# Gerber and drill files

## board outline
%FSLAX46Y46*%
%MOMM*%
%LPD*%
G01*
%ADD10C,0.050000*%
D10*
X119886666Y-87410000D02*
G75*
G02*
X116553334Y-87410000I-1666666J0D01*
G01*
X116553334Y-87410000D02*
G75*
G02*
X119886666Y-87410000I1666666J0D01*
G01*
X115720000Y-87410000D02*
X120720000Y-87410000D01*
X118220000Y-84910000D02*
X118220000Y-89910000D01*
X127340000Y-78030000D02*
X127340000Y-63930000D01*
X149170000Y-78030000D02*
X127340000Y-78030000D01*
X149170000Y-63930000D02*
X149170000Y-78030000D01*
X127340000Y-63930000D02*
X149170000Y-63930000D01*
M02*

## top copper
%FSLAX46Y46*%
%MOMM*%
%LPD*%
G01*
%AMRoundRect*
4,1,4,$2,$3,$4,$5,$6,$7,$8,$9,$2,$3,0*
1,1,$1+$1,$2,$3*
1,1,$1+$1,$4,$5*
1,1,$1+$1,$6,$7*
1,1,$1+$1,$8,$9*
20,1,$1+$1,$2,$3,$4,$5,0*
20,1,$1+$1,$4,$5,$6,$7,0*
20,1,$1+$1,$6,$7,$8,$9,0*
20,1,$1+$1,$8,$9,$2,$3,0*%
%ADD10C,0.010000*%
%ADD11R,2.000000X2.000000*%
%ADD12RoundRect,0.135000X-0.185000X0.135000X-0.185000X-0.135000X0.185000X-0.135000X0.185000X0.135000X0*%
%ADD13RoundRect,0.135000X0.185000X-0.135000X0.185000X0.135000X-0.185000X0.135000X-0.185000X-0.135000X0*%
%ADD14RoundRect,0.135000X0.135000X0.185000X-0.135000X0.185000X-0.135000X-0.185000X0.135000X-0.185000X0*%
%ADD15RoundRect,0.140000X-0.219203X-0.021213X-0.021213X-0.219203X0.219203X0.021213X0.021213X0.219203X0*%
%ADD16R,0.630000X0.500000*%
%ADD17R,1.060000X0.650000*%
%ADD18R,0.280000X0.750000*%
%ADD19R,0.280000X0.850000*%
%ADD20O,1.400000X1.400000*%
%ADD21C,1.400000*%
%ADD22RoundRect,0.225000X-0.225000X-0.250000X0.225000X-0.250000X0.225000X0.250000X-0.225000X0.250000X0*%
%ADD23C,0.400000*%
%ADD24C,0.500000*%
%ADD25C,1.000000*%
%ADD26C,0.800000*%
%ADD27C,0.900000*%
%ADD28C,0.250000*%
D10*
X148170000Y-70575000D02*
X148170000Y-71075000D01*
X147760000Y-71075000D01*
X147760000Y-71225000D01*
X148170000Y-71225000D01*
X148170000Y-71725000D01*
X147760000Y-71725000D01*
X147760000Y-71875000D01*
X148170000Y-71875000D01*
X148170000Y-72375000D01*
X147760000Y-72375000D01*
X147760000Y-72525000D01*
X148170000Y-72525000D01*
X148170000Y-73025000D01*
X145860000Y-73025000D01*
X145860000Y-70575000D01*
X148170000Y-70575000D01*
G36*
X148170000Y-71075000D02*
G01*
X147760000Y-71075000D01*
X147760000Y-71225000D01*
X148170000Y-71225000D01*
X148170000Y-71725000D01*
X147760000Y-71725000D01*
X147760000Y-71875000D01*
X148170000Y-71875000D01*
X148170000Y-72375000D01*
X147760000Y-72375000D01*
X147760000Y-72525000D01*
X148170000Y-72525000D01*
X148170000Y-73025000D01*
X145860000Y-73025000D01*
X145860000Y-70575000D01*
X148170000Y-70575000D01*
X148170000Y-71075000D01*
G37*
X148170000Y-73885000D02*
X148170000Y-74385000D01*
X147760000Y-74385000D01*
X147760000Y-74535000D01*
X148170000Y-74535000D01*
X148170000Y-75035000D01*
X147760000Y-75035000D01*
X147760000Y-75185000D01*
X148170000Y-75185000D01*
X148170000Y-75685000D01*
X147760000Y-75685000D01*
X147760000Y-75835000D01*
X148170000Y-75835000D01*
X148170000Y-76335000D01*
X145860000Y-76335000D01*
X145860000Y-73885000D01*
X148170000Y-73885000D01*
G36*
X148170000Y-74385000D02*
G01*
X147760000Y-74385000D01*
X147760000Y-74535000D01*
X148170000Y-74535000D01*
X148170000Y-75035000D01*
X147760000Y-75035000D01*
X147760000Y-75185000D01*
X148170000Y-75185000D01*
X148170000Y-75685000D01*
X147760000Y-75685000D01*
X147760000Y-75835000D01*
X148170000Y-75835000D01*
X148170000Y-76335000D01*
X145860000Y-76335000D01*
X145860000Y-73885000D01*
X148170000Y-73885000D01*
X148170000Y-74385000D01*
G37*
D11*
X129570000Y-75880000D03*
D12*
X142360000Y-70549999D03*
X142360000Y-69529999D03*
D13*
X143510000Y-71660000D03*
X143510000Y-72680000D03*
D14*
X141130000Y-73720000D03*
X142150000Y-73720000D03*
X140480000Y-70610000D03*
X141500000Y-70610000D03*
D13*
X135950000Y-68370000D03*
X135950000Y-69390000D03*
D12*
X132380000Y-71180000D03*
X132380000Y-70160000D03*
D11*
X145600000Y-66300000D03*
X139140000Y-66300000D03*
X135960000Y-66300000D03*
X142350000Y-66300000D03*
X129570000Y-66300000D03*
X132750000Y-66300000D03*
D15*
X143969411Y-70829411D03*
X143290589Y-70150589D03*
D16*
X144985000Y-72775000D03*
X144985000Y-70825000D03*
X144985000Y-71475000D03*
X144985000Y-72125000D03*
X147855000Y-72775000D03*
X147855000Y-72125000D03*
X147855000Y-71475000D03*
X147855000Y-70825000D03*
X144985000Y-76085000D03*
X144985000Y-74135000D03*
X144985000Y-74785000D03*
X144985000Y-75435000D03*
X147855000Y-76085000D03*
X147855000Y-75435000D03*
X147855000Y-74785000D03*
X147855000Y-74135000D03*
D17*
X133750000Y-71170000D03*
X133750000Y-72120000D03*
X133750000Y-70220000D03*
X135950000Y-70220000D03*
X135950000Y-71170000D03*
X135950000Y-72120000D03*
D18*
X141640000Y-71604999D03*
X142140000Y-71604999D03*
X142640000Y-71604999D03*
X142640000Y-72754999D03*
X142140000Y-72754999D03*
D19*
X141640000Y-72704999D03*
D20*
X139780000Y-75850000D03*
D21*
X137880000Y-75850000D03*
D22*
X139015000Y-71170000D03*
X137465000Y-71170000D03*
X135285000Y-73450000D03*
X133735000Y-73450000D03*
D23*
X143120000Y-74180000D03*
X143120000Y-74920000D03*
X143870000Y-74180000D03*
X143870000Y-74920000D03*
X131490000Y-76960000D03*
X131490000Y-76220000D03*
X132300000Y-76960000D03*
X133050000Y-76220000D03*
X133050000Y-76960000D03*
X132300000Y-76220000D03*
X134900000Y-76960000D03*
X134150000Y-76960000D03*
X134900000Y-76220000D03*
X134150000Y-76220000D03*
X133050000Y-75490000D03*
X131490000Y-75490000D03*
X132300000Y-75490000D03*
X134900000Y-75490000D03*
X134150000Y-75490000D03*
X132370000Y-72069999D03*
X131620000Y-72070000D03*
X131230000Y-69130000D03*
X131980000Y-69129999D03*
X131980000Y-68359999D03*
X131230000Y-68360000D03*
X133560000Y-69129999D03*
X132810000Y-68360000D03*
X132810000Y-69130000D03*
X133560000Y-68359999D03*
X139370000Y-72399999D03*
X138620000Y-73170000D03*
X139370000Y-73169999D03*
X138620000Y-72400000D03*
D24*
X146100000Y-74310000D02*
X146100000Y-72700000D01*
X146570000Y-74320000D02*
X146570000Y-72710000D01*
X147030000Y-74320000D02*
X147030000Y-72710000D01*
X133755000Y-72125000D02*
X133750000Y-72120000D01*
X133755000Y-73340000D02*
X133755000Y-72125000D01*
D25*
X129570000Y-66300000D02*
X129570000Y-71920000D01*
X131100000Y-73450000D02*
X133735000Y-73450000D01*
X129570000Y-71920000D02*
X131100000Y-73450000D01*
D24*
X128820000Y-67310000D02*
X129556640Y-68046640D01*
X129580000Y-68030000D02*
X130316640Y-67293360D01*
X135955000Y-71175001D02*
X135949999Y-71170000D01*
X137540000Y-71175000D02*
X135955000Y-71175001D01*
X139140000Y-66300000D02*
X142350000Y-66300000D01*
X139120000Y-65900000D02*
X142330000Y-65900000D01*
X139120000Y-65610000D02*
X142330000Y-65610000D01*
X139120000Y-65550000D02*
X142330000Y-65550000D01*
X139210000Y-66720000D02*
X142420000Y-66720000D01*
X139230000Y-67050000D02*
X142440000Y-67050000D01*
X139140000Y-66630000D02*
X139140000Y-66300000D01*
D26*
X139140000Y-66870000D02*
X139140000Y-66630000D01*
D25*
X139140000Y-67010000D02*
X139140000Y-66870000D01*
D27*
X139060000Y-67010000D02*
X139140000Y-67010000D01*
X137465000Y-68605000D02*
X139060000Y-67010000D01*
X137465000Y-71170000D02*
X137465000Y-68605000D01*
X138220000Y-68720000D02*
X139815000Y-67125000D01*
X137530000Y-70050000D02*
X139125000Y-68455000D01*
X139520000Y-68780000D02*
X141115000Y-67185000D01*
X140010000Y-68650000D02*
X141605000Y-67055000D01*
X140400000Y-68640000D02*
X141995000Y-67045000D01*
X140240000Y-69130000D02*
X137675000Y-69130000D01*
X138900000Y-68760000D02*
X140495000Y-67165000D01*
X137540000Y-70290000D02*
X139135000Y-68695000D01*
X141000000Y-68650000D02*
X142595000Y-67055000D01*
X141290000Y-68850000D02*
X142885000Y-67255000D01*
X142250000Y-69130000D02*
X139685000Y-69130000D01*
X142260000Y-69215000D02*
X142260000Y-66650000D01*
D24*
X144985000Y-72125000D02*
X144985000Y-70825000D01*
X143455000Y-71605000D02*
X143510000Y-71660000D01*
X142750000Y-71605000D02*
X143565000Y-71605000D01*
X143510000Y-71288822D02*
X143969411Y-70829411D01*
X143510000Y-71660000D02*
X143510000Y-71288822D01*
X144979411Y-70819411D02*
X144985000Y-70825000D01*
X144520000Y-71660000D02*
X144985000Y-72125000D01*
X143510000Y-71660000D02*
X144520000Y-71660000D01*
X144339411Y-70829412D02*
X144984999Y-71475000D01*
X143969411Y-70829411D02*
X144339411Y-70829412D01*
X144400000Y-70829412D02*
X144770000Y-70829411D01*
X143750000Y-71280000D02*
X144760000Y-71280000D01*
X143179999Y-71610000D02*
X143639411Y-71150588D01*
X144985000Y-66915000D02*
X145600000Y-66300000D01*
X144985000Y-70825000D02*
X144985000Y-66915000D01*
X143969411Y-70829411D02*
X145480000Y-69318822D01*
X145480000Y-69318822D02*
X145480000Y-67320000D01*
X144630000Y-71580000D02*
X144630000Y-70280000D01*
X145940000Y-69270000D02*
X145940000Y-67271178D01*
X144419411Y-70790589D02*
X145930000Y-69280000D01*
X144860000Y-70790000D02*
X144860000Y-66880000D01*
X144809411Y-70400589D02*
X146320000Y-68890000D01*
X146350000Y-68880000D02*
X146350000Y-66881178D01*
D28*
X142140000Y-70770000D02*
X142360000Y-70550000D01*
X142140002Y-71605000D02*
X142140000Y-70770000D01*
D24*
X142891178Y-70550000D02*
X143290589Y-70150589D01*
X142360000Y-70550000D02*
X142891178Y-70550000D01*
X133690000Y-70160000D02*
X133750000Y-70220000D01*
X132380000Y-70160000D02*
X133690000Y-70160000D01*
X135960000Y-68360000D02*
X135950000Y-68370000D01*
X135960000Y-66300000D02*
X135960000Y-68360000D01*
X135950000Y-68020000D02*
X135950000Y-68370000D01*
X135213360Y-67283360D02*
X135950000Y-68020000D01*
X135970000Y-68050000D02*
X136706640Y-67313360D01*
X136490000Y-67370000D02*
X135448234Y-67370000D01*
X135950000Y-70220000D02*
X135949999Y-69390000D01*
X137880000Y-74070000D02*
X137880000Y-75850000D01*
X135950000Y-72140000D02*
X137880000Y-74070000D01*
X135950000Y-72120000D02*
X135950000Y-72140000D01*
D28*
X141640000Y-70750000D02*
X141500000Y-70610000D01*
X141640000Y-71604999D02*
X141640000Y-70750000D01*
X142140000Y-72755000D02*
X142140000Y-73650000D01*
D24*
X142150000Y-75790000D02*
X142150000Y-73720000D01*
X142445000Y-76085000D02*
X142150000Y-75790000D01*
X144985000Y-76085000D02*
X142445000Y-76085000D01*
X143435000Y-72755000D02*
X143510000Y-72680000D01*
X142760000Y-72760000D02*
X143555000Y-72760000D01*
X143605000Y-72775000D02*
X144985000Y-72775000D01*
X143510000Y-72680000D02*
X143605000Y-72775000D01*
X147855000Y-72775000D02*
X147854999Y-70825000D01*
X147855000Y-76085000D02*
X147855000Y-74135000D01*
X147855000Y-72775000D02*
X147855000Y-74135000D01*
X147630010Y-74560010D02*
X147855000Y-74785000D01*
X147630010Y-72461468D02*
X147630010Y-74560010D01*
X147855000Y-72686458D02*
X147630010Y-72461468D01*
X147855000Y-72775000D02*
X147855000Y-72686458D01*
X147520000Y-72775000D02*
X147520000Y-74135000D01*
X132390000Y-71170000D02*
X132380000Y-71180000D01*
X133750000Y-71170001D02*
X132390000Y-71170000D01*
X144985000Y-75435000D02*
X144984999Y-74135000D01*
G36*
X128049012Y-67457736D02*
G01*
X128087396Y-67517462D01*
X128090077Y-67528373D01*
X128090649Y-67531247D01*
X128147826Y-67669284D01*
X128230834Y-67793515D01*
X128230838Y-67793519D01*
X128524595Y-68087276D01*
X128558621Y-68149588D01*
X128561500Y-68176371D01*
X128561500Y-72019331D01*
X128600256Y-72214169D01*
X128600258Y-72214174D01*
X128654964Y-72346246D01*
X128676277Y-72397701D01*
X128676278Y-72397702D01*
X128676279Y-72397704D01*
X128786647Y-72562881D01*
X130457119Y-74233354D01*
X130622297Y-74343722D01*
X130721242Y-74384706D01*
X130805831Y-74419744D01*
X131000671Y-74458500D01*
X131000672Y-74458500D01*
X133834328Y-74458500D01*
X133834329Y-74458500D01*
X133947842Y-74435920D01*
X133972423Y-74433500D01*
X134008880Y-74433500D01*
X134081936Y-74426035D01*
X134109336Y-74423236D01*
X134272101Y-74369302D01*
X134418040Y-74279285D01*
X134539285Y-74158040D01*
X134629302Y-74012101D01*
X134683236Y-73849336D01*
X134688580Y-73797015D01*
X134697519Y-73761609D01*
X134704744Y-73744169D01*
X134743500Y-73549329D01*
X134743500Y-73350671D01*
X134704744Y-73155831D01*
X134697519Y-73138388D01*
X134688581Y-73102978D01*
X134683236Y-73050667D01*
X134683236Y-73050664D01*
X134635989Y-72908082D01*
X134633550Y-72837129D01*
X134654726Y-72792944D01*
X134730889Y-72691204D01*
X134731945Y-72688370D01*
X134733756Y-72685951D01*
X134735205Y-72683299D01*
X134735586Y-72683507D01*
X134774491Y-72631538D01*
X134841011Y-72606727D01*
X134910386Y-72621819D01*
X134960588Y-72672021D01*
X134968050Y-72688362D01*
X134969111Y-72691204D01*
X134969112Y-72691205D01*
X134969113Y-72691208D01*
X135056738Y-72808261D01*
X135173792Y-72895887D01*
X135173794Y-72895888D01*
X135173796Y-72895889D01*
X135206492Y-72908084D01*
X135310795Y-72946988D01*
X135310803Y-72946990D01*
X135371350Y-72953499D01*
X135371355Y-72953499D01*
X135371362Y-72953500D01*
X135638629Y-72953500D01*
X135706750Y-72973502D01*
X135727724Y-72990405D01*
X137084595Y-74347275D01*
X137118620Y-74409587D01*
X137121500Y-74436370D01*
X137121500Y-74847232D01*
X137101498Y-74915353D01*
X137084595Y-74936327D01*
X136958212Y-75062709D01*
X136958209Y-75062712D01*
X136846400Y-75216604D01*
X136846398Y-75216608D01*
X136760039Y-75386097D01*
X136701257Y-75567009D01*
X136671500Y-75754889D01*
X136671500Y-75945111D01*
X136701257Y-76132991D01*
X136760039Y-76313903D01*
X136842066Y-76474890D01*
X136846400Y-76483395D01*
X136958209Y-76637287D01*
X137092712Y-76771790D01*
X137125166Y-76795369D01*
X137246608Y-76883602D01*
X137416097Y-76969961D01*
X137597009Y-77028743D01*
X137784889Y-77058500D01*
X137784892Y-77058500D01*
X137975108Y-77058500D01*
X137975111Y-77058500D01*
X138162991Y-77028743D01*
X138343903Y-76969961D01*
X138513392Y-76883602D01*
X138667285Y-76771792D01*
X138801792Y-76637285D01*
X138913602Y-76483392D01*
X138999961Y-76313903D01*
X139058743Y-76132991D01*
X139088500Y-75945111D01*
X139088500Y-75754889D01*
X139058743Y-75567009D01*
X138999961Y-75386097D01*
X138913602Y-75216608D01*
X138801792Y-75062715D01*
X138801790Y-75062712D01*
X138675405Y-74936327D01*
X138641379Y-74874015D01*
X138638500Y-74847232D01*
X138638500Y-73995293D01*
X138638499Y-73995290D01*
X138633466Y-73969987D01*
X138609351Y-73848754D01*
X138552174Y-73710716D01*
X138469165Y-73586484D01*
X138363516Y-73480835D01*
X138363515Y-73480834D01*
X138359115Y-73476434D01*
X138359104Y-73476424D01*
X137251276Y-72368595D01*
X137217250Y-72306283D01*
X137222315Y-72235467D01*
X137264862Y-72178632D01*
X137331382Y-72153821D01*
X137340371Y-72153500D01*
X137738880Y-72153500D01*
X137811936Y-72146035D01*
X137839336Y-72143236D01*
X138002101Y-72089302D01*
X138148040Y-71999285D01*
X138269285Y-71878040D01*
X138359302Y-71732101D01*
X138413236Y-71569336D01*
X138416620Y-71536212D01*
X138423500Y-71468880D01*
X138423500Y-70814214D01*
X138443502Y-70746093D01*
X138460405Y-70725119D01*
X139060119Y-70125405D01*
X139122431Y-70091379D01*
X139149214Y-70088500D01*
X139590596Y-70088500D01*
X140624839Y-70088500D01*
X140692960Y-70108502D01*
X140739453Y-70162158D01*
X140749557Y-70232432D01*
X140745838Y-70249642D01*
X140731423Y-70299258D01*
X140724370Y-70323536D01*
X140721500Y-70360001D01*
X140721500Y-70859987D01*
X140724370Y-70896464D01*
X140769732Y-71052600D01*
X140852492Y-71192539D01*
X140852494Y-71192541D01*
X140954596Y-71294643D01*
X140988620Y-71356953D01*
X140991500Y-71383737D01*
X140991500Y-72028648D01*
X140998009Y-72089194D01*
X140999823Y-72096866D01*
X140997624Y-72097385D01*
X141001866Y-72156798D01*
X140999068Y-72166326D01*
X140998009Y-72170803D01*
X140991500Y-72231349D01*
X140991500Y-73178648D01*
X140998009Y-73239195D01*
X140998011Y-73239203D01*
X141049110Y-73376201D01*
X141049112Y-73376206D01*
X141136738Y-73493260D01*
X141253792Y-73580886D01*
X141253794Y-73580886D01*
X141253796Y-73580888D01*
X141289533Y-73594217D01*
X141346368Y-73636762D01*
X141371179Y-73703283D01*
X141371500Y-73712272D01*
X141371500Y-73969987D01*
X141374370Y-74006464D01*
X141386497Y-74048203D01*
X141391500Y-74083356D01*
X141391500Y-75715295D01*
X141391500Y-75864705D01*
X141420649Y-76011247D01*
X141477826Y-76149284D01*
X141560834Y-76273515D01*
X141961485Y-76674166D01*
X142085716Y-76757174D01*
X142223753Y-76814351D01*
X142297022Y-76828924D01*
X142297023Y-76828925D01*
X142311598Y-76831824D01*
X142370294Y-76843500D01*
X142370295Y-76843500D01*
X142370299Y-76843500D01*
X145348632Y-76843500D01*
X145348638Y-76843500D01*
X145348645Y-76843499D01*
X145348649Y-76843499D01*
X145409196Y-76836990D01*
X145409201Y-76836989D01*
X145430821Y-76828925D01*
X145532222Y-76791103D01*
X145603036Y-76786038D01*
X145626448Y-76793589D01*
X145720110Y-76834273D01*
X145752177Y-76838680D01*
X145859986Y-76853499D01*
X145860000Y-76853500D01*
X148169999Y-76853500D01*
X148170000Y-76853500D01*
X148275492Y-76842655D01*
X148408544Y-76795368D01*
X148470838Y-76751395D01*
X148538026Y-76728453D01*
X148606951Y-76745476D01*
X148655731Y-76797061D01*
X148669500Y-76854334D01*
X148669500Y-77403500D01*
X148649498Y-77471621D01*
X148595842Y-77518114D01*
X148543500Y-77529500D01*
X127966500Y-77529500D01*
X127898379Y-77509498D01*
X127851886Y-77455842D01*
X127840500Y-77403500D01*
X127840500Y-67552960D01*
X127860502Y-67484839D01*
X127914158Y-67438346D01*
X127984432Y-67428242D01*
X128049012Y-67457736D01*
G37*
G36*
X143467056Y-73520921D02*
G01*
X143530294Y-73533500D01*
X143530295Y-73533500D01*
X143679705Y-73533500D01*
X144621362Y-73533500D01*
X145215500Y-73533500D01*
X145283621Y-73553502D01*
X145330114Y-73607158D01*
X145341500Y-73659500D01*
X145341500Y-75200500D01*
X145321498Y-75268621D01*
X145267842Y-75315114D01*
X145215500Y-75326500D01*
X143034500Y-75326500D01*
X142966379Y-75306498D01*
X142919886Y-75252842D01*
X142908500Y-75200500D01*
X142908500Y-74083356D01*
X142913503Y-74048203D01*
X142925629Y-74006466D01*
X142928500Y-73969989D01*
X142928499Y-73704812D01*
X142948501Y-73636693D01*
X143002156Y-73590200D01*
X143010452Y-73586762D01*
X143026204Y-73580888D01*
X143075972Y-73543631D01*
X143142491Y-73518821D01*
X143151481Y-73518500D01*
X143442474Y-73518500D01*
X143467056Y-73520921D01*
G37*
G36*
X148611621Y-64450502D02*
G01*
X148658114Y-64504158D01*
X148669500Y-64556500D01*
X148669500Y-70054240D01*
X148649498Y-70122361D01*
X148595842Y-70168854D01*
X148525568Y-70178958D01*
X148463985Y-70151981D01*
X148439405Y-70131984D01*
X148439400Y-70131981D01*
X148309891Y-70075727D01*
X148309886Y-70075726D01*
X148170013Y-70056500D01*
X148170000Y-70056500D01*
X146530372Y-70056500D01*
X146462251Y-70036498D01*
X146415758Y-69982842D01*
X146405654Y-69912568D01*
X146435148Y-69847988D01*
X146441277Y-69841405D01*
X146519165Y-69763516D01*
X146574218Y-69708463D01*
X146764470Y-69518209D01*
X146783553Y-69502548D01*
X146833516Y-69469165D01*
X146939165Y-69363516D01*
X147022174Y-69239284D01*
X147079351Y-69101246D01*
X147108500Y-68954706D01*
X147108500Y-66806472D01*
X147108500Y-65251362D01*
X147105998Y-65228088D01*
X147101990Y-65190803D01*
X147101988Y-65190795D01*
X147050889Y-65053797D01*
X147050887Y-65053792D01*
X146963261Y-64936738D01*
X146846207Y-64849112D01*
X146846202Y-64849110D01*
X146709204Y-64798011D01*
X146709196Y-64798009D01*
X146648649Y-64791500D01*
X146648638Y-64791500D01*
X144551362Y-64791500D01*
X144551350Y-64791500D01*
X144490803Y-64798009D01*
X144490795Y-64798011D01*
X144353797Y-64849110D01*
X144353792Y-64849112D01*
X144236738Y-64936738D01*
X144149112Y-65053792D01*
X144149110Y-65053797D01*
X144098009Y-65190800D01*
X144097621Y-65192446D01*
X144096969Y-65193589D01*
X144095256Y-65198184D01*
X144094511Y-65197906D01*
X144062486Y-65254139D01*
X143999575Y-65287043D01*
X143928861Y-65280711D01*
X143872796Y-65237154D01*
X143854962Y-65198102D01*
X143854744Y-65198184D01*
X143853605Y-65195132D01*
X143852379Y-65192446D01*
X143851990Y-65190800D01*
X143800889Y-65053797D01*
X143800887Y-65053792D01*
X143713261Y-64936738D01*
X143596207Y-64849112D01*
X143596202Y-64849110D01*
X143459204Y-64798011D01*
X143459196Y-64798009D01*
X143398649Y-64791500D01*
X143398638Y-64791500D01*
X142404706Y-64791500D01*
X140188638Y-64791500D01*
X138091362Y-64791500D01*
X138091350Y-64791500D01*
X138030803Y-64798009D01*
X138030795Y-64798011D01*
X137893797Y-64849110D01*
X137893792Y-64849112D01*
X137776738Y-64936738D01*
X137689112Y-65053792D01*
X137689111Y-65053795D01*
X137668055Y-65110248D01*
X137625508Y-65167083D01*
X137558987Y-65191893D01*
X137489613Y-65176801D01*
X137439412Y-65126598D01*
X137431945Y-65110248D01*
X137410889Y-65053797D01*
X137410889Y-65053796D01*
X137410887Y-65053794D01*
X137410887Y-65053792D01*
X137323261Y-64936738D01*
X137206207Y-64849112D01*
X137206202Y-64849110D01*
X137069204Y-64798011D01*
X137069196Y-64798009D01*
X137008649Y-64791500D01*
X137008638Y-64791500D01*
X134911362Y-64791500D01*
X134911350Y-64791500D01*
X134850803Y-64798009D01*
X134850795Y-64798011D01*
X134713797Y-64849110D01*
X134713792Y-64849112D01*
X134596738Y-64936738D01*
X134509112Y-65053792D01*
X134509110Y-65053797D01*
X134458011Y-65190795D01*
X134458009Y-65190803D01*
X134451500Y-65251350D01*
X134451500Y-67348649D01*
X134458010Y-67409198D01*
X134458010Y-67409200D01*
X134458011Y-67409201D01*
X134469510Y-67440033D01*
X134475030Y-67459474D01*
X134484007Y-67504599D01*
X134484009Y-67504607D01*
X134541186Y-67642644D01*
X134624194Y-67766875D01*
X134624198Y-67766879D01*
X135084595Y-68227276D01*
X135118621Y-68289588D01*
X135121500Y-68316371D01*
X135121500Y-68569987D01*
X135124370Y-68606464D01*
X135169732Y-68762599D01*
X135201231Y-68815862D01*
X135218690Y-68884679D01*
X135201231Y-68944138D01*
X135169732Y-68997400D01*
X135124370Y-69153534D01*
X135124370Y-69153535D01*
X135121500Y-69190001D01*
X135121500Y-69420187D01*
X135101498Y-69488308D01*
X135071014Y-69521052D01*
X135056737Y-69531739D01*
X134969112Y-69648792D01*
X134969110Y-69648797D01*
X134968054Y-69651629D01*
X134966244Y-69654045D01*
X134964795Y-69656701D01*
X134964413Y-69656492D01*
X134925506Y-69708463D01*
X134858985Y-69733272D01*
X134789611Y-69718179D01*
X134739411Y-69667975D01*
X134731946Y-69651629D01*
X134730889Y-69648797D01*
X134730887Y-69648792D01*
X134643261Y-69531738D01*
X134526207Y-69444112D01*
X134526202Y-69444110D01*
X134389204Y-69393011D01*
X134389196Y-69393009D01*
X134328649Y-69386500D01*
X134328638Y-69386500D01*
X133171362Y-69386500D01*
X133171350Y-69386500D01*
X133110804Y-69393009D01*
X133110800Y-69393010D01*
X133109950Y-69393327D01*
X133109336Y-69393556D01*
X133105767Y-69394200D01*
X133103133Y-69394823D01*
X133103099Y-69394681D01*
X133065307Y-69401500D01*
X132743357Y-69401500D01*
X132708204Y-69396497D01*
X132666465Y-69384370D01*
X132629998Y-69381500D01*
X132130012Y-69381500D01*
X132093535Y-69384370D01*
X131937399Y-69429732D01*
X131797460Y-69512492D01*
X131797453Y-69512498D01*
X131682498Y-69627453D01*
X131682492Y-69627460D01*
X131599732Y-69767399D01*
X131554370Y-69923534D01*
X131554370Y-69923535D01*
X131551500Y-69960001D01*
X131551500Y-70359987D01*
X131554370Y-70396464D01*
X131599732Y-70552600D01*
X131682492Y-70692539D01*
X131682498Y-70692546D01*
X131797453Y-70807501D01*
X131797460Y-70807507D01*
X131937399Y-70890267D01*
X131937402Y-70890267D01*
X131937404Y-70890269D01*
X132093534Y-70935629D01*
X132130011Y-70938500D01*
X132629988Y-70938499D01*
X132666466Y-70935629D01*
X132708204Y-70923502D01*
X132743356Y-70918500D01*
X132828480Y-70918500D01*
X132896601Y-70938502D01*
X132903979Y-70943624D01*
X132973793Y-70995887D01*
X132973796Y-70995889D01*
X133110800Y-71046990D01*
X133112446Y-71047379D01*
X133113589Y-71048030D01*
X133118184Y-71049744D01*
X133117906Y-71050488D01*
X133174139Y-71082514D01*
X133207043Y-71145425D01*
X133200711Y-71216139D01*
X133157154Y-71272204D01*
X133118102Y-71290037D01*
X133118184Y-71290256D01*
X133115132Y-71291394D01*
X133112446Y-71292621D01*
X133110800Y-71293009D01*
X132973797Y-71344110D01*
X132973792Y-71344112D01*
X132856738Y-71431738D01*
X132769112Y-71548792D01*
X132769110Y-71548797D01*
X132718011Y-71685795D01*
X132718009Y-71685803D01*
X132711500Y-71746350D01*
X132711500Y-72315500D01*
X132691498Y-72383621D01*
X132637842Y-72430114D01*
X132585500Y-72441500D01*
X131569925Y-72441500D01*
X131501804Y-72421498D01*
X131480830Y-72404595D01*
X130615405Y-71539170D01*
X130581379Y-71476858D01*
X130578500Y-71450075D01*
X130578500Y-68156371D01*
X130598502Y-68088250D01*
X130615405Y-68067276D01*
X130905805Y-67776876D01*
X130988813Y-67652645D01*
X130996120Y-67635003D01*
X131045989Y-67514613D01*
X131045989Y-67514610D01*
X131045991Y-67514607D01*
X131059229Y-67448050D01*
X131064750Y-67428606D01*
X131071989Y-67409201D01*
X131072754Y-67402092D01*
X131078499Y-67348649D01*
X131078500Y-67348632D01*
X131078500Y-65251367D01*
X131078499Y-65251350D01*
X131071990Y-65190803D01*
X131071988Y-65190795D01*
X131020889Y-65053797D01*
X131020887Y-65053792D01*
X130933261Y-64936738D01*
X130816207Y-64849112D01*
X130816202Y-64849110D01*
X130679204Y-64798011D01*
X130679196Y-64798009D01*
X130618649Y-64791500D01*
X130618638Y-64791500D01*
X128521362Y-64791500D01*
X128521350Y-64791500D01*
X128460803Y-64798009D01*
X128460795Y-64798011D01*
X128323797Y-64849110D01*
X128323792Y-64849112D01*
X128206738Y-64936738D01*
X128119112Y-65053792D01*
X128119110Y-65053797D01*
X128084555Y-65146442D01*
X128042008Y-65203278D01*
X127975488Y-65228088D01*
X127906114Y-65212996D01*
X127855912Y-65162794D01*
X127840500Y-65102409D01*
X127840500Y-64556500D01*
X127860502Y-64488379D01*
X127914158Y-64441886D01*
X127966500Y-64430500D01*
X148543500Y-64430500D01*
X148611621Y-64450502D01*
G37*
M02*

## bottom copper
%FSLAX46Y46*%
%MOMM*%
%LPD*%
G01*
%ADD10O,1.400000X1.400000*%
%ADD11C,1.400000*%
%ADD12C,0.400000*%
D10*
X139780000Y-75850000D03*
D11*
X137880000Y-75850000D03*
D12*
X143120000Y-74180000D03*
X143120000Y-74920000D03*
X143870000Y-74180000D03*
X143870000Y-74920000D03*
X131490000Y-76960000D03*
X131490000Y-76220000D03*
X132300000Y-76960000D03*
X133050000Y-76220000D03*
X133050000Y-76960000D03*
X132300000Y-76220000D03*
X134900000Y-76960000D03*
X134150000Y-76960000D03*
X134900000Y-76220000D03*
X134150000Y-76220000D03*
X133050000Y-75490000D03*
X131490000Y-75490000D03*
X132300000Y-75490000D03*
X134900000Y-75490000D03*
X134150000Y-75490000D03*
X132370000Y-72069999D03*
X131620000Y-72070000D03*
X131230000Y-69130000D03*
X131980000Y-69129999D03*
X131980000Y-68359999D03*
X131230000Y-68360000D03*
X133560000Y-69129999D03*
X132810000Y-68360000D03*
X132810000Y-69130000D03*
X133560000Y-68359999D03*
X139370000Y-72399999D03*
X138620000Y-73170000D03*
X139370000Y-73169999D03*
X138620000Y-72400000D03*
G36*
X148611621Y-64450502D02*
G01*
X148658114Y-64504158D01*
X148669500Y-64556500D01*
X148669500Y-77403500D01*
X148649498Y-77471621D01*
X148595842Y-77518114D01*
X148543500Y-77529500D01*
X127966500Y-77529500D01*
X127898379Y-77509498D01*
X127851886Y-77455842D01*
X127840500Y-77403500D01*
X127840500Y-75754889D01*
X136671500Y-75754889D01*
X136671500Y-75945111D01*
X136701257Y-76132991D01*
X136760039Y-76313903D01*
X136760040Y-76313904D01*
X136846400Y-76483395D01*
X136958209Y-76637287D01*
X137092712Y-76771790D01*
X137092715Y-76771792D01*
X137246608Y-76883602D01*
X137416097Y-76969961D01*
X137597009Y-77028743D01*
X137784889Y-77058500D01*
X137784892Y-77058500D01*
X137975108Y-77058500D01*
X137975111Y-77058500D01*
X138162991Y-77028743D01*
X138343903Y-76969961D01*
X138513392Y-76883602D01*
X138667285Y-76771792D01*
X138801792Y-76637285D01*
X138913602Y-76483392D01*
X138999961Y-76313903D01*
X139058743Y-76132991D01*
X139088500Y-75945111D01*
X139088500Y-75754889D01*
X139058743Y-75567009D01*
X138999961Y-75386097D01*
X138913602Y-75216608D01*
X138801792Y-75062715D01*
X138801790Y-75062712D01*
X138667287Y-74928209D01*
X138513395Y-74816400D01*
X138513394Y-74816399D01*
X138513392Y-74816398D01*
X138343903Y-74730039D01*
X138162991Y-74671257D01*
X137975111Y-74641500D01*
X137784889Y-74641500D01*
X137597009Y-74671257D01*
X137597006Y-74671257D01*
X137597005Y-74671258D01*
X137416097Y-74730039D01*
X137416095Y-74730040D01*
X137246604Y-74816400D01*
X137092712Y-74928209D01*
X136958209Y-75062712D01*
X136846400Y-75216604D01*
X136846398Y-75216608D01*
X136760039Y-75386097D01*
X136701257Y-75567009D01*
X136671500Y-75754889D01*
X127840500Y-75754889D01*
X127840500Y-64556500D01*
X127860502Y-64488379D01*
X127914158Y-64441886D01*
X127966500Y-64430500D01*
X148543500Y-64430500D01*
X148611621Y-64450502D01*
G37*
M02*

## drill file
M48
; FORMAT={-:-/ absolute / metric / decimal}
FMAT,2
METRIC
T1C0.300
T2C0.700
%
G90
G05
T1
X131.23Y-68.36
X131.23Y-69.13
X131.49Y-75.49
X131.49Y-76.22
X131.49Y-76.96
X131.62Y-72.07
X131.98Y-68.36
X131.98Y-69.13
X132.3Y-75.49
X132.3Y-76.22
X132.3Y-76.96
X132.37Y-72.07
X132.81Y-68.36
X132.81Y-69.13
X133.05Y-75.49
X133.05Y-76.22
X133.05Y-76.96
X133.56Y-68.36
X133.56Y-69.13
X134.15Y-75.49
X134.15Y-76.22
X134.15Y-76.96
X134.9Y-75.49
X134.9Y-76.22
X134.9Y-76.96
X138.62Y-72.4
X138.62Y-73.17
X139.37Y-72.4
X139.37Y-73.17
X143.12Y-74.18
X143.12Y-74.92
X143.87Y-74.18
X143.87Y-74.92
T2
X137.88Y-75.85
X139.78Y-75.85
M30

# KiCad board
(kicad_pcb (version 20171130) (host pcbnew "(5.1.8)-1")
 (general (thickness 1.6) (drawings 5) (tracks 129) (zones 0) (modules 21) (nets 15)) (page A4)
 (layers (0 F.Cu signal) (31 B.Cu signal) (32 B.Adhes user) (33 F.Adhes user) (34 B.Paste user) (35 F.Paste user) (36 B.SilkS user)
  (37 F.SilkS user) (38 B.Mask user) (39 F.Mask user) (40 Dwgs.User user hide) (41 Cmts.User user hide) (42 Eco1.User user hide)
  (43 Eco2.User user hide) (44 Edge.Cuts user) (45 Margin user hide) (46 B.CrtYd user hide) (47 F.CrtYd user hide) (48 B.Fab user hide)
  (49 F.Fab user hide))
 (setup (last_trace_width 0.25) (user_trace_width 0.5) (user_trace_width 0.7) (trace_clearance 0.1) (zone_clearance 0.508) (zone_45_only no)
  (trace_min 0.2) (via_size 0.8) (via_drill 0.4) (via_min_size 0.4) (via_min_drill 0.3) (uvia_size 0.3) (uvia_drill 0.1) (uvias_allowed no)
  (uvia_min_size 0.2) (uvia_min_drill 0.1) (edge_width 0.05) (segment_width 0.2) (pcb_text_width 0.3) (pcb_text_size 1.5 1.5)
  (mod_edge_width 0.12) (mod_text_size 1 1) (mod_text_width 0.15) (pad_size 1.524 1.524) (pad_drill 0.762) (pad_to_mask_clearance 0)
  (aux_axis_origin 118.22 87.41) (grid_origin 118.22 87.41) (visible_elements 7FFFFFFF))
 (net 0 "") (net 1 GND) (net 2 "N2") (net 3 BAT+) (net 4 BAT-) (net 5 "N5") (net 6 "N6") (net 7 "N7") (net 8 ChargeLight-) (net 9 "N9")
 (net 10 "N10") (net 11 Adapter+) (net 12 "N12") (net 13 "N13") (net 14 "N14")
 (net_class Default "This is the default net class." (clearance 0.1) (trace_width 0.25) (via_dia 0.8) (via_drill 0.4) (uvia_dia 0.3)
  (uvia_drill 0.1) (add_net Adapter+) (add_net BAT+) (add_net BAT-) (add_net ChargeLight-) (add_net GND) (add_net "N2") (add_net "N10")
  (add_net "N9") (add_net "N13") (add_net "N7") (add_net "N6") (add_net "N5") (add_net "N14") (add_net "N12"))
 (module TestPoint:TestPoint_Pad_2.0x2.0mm (layer F.Cu) (at 129.57 75.88 180)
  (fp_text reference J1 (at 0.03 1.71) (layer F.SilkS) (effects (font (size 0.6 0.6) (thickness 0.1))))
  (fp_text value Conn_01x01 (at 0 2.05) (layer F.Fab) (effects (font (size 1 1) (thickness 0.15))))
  (pad 1 smd rect (at 0 0 180) (size 2 2) (layers F.Cu F.Mask) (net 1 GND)))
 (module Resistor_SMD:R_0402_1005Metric (layer F.Cu) (at 142.36 70.039999 270)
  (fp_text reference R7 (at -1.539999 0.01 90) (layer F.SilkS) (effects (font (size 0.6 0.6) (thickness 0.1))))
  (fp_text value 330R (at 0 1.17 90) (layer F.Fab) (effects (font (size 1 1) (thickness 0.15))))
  (pad 2 smd roundrect (at 0.51 0 270) (size 0.54 0.64) (layers F.Cu F.Paste F.Mask) (roundrect_rratio 0.25) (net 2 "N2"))
  (pad 1 smd roundrect (at -0.51 0 270) (size 0.54 0.64) (layers F.Cu F.Paste F.Mask) (roundrect_rratio 0.25) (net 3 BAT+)))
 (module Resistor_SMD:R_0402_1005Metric (layer F.Cu) (at 143.51 72.17 90)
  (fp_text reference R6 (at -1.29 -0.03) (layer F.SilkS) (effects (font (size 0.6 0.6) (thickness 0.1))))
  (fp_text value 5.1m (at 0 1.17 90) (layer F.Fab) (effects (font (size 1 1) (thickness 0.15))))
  (pad 2 smd roundrect (at 0.51 0 90) (size 0.54 0.64) (layers F.Cu F.Paste F.Mask) (roundrect_rratio 0.25) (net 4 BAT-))
  (pad 1 smd roundrect (at -0.51 0 90) (size 0.54 0.64) (layers F.Cu F.Paste F.Mask) (roundrect_rratio 0.25) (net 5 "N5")))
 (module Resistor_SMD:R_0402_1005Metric (layer F.Cu) (at 141.64 73.72 180)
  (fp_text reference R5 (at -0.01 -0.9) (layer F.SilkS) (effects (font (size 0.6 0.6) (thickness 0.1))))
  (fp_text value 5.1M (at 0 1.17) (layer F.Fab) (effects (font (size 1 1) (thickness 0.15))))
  (pad 2 smd roundrect (at 0.51 0 180) (size 0.54 0.64) (layers F.Cu F.Paste F.Mask) (roundrect_rratio 0.25) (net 1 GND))
  (pad 1 smd roundrect (at -0.51 0 180) (size 0.54 0.64) (layers F.Cu F.Paste F.Mask) (roundrect_rratio 0.25) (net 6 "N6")))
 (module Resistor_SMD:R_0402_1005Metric (layer F.Cu) (at 140.99 70.61 180)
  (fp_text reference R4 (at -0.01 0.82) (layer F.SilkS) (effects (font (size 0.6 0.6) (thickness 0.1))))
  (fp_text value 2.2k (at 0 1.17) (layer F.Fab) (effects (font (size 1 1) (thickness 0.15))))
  (pad 2 smd roundrect (at 0.51 0 180) (size 0.54 0.64) (layers F.Cu F.Paste F.Mask) (roundrect_rratio 0.25) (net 1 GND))
  (pad 1 smd roundrect (at -0.51 0 180) (size 0.54 0.64) (layers F.Cu F.Paste F.Mask) (roundrect_rratio 0.25) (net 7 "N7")))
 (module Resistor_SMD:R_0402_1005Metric (layer F.Cu) (at 135.95 68.88 90)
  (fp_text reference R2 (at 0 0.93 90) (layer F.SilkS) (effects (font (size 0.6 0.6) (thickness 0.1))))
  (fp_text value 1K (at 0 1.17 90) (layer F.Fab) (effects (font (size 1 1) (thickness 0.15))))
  (pad 2 smd roundrect (at 0.51 0 90) (size 0.54 0.64) (layers F.Cu F.Paste F.Mask) (roundrect_rratio 0.25) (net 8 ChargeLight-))
  (pad 1 smd roundrect (at -0.51 0 90) (size 0.54 0.64) (layers F.Cu F.Paste F.Mask) (roundrect_rratio 0.25) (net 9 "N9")))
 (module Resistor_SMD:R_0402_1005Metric (layer F.Cu) (at 132.38 70.67 270)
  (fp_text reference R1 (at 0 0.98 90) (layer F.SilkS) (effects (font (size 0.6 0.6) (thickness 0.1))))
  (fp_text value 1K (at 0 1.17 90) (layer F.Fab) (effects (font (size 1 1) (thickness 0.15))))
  (pad 2 smd roundrect (at 0.51 0 270) (size 0.54 0.64) (layers F.Cu F.Paste F.Mask) (roundrect_rratio 0.25) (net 1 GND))
  (pad 1 smd roundrect (at -0.51 0 270) (size 0.54 0.64) (layers F.Cu F.Paste F.Mask) (roundrect_rratio 0.25) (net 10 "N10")))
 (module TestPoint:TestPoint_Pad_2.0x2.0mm (layer F.Cu) (at 145.6 66.3 180)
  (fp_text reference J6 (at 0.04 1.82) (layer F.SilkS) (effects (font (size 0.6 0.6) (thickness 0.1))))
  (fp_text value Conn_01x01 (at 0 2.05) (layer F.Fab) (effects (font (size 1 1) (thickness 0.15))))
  (pad 1 smd rect (at 0 0 180) (size 2 2) (layers F.Cu F.Mask) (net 4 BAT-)))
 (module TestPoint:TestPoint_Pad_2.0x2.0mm (layer F.Cu) (at 139.14 66.3 180)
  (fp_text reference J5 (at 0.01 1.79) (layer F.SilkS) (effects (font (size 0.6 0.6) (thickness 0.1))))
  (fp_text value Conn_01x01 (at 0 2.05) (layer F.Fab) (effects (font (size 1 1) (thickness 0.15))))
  (pad 1 smd rect (at 0 0 180) (size 2 2) (layers F.Cu F.Mask) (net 3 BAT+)))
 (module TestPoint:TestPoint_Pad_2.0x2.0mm (layer F.Cu) (at 135.96 66.3 180)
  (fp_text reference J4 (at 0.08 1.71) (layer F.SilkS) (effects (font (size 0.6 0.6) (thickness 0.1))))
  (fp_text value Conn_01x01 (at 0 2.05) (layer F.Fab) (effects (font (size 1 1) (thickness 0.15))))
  (pad 1 smd rect (at 0 0 180) (size 2 2) (layers F.Cu F.Mask) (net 8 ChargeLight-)))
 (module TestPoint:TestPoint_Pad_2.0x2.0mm (layer F.Cu) (at 142.35 66.3 180)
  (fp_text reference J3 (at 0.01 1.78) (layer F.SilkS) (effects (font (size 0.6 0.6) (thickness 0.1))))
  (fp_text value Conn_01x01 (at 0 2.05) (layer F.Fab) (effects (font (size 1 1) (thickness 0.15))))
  (pad 1 smd rect (at 0 0 180) (size 2 2) (layers F.Cu F.Mask) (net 3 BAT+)))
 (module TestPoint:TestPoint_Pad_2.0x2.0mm (layer F.Cu) (at 129.57 66.3 180)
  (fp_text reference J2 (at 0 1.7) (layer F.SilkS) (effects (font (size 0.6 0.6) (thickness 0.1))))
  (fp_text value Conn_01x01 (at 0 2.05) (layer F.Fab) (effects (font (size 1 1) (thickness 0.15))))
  (pad 1 smd rect (at 0 0 180) (size 2 2) (layers F.Cu F.Mask) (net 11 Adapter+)))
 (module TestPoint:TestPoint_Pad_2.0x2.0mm (layer F.Cu) (at 132.75 66.3 180)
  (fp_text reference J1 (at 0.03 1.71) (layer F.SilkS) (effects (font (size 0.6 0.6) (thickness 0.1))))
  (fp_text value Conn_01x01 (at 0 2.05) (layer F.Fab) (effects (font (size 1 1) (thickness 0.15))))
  (pad 1 smd rect (at 0 0 180) (size 2 2) (layers F.Cu F.Mask) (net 1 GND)))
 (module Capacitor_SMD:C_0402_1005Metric (layer F.Cu) (at 143.63 70.49 315)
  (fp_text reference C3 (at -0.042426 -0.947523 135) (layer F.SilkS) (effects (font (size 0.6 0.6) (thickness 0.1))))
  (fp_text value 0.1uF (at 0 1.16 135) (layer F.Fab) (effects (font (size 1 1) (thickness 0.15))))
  (pad 2 smd roundrect (at 0.48 0 315) (size 0.56 0.62) (layers F.Cu F.Paste F.Mask) (roundrect_rratio 0.25) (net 4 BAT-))
  (pad 1 smd roundrect (at -0.48 0 315) (size 0.56 0.62) (layers F.Cu F.Paste F.Mask) (roundrect_rratio 0.25) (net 2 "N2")))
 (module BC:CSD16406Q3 (layer F.Cu) (at 146.42 71.8)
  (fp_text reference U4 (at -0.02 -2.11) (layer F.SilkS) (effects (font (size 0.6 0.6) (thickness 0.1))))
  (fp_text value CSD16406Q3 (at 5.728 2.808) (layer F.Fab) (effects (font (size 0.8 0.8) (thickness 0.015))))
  (fp_poly
   (pts (xy 1.75 -1.225) (xy 1.75 -0.725) (xy 1.34 -0.725) (xy 1.34 -0.575) (xy 1.75 -0.575) (xy 1.75 -0.075) (xy 1.34 -0.075)
    (xy 1.34 0.075) (xy 1.75 0.075) (xy 1.75 0.575) (xy 1.34 0.575) (xy 1.34 0.725) (xy 1.75 0.725) (xy 1.75 1.225) (xy -0.56 1.225)
    (xy -0.56 -1.225))
   (layer F.Cu) (width 0.01))
  (pad 4 smd rect (at -1.435 0.975) (size 0.63 0.5) (layers F.Cu F.Mask) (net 5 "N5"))
  (pad 1 smd rect (at -1.435 -0.975) (size 0.63 0.5) (layers F.Cu F.Mask) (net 4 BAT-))
  (pad 2 smd rect (at -1.435 -0.325) (size 0.63 0.5) (layers F.Cu F.Mask) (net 4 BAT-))
  (pad 3 smd rect (at -1.435 0.325) (size 0.63 0.5) (layers F.Cu F.Mask) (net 4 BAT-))
  (pad 5 smd rect (at 1.435 0.975) (size 0.63 0.5) (layers F.Cu) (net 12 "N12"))
  (pad 6 smd rect (at 1.435 0.325) (size 0.63 0.5) (layers F.Cu) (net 12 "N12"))
  (pad 7 smd rect (at 1.435 -0.325) (size 0.63 0.5) (layers F.Cu) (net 12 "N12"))
  (pad 8 smd rect (at 1.435 -0.975) (size 0.63 0.5) (layers F.Cu) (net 12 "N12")))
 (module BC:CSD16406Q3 (layer F.Cu) (at 146.42 75.11)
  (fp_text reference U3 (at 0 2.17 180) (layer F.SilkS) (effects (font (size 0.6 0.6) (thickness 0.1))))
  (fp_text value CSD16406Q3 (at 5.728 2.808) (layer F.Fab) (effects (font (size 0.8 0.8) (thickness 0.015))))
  (fp_poly
   (pts (xy 1.75 -1.225) (xy 1.75 -0.725) (xy 1.34 -0.725) (xy 1.34 -0.575) (xy 1.75 -0.575) (xy 1.75 -0.075) (xy 1.34 -0.075)
    (xy 1.34 0.075) (xy 1.75 0.075) (xy 1.75 0.575) (xy 1.34 0.575) (xy 1.34 0.725) (xy 1.75 0.725) (xy 1.75 1.225) (xy -0.56 1.225)
    (xy -0.56 -1.225))
   (layer F.Cu) (width 0.01))
  (pad 4 smd rect (at -1.435 0.975) (size 0.63 0.5) (layers F.Cu F.Mask) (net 6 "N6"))
  (pad 1 smd rect (at -1.435 -0.975) (size 0.63 0.5) (layers F.Cu F.Mask) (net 1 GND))
  (pad 2 smd rect (at -1.435 -0.325) (size 0.63 0.5) (layers F.Cu F.Mask) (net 1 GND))
  (pad 3 smd rect (at -1.435 0.325) (size 0.63 0.5) (layers F.Cu F.Mask) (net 1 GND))
  (pad 5 smd rect (at 1.435 0.975) (size 0.63 0.5) (layers F.Cu) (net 12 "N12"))
  (pad 6 smd rect (at 1.435 0.325) (size 0.63 0.5) (layers F.Cu) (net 12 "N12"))
  (pad 7 smd rect (at 1.435 -0.325) (size 0.63 0.5) (layers F.Cu) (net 12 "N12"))
  (pad 8 smd rect (at 1.435 -0.975) (size 0.63 0.5) (layers F.Cu) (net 12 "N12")))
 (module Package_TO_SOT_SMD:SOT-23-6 (layer F.Cu) (at 134.85 71.17 180)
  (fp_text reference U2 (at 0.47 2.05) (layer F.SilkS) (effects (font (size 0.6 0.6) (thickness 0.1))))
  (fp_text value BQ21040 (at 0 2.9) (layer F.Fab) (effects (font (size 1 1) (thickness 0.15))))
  (pad 5 smd rect (at 1.1 0 180) (size 1.06 0.65) (layers F.Cu F.Paste F.Mask) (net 1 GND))
  (pad 6 smd rect (at 1.1 -0.95 180) (size 1.06 0.65) (layers F.Cu F.Paste F.Mask) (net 11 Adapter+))
  (pad 4 smd rect (at 1.1 0.95 180) (size 1.06 0.65) (layers F.Cu F.Paste F.Mask) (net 10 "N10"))
  (pad 3 smd rect (at -1.1 0.95 180) (size 1.06 0.65) (layers F.Cu F.Paste F.Mask) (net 9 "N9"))
  (pad 2 smd rect (at -1.1 0 180) (size 1.06 0.65) (layers F.Cu F.Paste F.Mask) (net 3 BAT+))
  (pad 1 smd rect (at -1.1 -0.95 180) (size 1.06 0.65) (layers F.Cu F.Paste F.Mask) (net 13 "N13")))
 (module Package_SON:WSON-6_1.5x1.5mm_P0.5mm (layer F.Cu) (at 142.14 72.179999 90)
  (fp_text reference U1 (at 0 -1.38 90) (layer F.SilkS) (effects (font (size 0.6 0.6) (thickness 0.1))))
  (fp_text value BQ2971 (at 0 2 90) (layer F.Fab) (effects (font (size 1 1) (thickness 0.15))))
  (pad 6 smd rect (at 0.575 -0.5) (size 0.28 0.75) (layers F.Cu F.Paste F.Mask) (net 7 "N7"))
  (pad 5 smd rect (at 0.575 0) (size 0.28 0.75) (layers F.Cu F.Paste F.Mask) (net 2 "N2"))
  (pad 4 smd rect (at 0.575 0.5) (size 0.28 0.75) (layers F.Cu F.Paste F.Mask) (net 4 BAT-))
  (pad 3 smd rect (at -0.575 0.5) (size 0.28 0.75) (layers F.Cu F.Paste F.Mask) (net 5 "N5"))
  (pad 2 smd rect (at -0.575 0) (size 0.28 0.75) (layers F.Cu F.Paste F.Mask) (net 6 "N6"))
  (pad 1 smd rect (at -0.525 -0.5) (size 0.28 0.85) (layers F.Cu F.Paste F.Mask) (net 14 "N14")))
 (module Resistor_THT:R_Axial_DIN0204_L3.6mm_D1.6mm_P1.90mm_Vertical (layer F.Cu) (at 137.88 75.85)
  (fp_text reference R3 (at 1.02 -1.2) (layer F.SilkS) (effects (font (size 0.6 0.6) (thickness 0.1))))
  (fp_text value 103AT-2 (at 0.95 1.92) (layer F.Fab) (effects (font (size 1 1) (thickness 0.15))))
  (pad 2 thru_hole oval (at 1.9 0) (size 1.4 1.4) (drill 0.7) (layers *.Cu *.Mask) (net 1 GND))
  (pad 1 thru_hole circle (at 0 0) (size 1.4 1.4) (drill 0.7) (layers *.Cu *.Mask) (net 13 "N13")))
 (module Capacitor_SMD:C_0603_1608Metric (layer F.Cu) (at 138.24 71.17)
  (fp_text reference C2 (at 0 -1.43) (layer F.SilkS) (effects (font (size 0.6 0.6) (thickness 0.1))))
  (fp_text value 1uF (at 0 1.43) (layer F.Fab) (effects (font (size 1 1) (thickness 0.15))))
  (pad 2 smd roundrect (at 0.775 0) (size 0.9 0.95) (layers F.Cu F.Paste F.Mask) (roundrect_rratio 0.25) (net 1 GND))
  (pad 1 smd roundrect (at -0.775 0) (size 0.9 0.95) (layers F.Cu F.Paste F.Mask) (roundrect_rratio 0.25) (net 3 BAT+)))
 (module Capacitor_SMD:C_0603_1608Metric (layer F.Cu) (at 134.51 73.45)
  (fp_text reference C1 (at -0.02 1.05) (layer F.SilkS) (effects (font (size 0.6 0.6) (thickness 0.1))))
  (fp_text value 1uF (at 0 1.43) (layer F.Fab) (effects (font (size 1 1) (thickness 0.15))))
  (pad 2 smd roundrect (at 0.775 0) (size 0.9 0.95) (layers F.Cu F.Paste F.Mask) (roundrect_rratio 0.25) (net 1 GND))
  (pad 1 smd roundrect (at -0.775 0) (size 0.9 0.95) (layers F.Cu F.Paste F.Mask) (roundrect_rratio 0.25) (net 11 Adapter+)))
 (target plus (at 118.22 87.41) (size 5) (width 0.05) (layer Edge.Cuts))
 (gr_line (start 127.34 78.03) (end 127.34 63.93) (layer Edge.Cuts) (width 0.05))
 (gr_line (start 149.17 78.03) (end 127.34 78.03) (layer Edge.Cuts) (width 0.05))
 (gr_line (start 149.17 63.93) (end 149.17 78.03) (layer Edge.Cuts) (width 0.05))
 (gr_line (start 127.34 63.93) (end 149.17 63.93) (layer Edge.Cuts) (width 0.05))
 (segment (start 146.1 74.31) (end 146.1 72.7) (width 0.5) (layer F.Cu) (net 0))
 (segment (start 146.57 74.32) (end 146.57 72.71) (width 0.5) (layer F.Cu) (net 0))
 (segment (start 147.03 74.32) (end 147.03 72.71) (width 0.5) (layer F.Cu) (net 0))
 (segment (start 133.755 72.125) (end 133.75 72.12) (width 0.5) (layer F.Cu) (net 11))
 (segment (start 133.755 73.34) (end 133.755 72.125) (width 0.5) (layer F.Cu) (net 11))
 (segment (start 129.57 66.3) (end 129.57 71.92) (width 1) (layer F.Cu) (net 11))
 (segment (start 131.1 73.45) (end 133.735 73.45) (width 1) (layer F.Cu) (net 11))
 (segment (start 129.57 71.92) (end 131.1 73.45) (width 1) (layer F.Cu) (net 11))
 (segment (start 128.82 67.31) (end 129.55664 68.04664) (width 0.5) (layer F.Cu) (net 11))
 (segment (start 129.58 68.03) (end 130.31664 67.29336) (width 0.5) (layer F.Cu) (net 11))
 (segment (start 135.955 71.175001) (end 135.949999 71.17) (width 0.5) (layer F.Cu) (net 3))
 (segment (start 137.54 71.175) (end 135.955 71.175001) (width 0.5) (layer F.Cu) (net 3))
 (segment (start 139.14 66.3) (end 142.35 66.3) (width 0.5) (layer F.Cu) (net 3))
 (segment (start 139.12 65.9) (end 142.33 65.9) (width 0.5) (layer F.Cu) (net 3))
 (segment (start 139.12 65.61) (end 142.33 65.61) (width 0.5) (layer F.Cu) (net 3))
 (segment (start 139.12 65.55) (end 142.33 65.55) (width 0.5) (layer F.Cu) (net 3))
 (segment (start 139.21 66.72) (end 142.42 66.72) (width 0.5) (layer F.Cu) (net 3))
 (segment (start 139.23 67.05) (end 142.44 67.05) (width 0.5) (layer F.Cu) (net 3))
 (segment (start 139.14 66.63) (end 139.14 66.3) (width 0.5) (layer F.Cu) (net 3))
 (segment (start 139.14 66.87) (end 139.14 66.63) (width 0.8) (layer F.Cu) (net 3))
 (segment (start 139.14 67.01) (end 139.14 66.87) (width 1) (layer F.Cu) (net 3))
 (segment (start 139.06 67.01) (end 139.14 67.01) (width 0.9) (layer F.Cu) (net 3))
 (segment (start 137.465 68.605) (end 139.06 67.01) (width 0.9) (layer F.Cu) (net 3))
 (segment (start 137.465 71.17) (end 137.465 68.605) (width 0.9) (layer F.Cu) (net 3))
 (segment (start 138.22 68.72) (end 139.815 67.125) (width 0.9) (layer F.Cu) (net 3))
 (segment (start 137.53 70.05) (end 139.125 68.455) (width 0.9) (layer F.Cu) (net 3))
 (segment (start 139.52 68.78) (end 141.115 67.185) (width 0.9) (layer F.Cu) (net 3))
 (segment (start 140.01 68.65) (end 141.605 67.055) (width 0.9) (layer F.Cu) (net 3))
 (segment (start 140.4 68.64) (end 141.995 67.045) (width 0.9) (layer F.Cu) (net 3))
 (segment (start 140.24 69.13) (end 137.675 69.13) (width 0.9) (layer F.Cu) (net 3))
 (segment (start 138.9 68.76) (end 140.495 67.165) (width 0.9) (layer F.Cu) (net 3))
 (segment (start 137.54 70.29) (end 139.135 68.695) (width 0.9) (layer F.Cu) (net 3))
 (segment (start 141 68.65) (end 142.595 67.055) (width 0.9) (layer F.Cu) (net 3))
 (segment (start 141.29 68.85) (end 142.885 67.255) (width 0.9) (layer F.Cu) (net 3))
 (segment (start 142.25 69.13) (end 139.685 69.13) (width 0.9) (layer F.Cu) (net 3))
 (segment (start 142.26 69.215) (end 142.26 66.65) (width 0.9) (layer F.Cu) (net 3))
 (segment (start 144.985 72.125) (end 144.985 70.825) (width 0.5) (layer F.Cu) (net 4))
 (segment (start 143.455 71.605) (end 143.51 71.66) (width 0.5) (layer F.Cu) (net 4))
 (segment (start 142.75 71.605) (end 143.565 71.605) (width 0.5) (layer F.Cu) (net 4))
 (segment (start 143.51 71.288822) (end 143.969411 70.829411) (width 0.5) (layer F.Cu) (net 4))
 (segment (start 143.51 71.66) (end 143.51 71.288822) (width 0.5) (layer F.Cu) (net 4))
 (segment (start 144.979411 70.819411) (end 144.985 70.825) (width 0.5) (layer F.Cu) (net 4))
 (segment (start 144.52 71.66) (end 144.985 72.125) (width 0.5) (layer F.Cu) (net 4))
 (segment (start 143.51 71.66) (end 144.52 71.66) (width 0.5) (layer F.Cu) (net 4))
 (segment (start 144.339411 70.829412) (end 144.984999 71.475) (width 0.5) (layer F.Cu) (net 4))
 (segment (start 143.969411 70.829411) (end 144.339411 70.829412) (width 0.5) (layer F.Cu) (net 4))
 (segment (start 144.4 70.829412) (end 144.77 70.829411) (width 0.5) (layer F.Cu) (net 4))
 (segment (start 143.75 71.28) (end 144.76 71.28) (width 0.5) (layer F.Cu) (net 4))
 (segment (start 143.179999 71.61) (end 143.639411 71.150588) (width 0.5) (layer F.Cu) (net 4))
 (segment (start 144.985 66.915) (end 145.6 66.3) (width 0.5) (layer F.Cu) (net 4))
 (segment (start 144.985 70.825) (end 144.985 66.915) (width 0.5) (layer F.Cu) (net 4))
 (segment (start 143.969411 70.829411) (end 145.48 69.318822) (width 0.5) (layer F.Cu) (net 4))
 (segment (start 145.48 69.318822) (end 145.48 67.32) (width 0.5) (layer F.Cu) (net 4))
 (segment (start 144.63 71.58) (end 144.63 70.28) (width 0.5) (layer F.Cu) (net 4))
 (segment (start 145.94 69.27) (end 145.94 67.271178) (width 0.5) (layer F.Cu) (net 4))
 (segment (start 144.419411 70.790589) (end 145.93 69.28) (width 0.5) (layer F.Cu) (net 4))
 (segment (start 144.86 70.79) (end 144.86 66.88) (width 0.5) (layer F.Cu) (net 4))
 (segment (start 144.809411 70.400589) (end 146.32 68.89) (width 0.5) (layer F.Cu) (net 4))
 (segment (start 146.35 68.88) (end 146.35 66.881178) (width 0.5) (layer F.Cu) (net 4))
 (segment (start 142.14 70.77) (end 142.36 70.55) (width 0.25) (layer F.Cu) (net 2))
 (segment (start 142.140002 71.605) (end 142.14 70.77) (width 0.25) (layer F.Cu) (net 2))
 (segment (start 142.891178 70.55) (end 143.290589 70.150589) (width 0.5) (layer F.Cu) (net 2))
 (segment (start 142.36 70.55) (end 142.891178 70.55) (width 0.5) (layer F.Cu) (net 2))
 (segment (start 133.69 70.16) (end 133.75 70.22) (width 0.5) (layer F.Cu) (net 10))
 (segment (start 132.38 70.16) (end 133.69 70.16) (width 0.5) (layer F.Cu) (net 10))
 (segment (start 135.96 68.36) (end 135.95 68.37) (width 0.5) (layer F.Cu) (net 8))
 (segment (start 135.96 66.3) (end 135.96 68.36) (width 0.5) (layer F.Cu) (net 8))
 (segment (start 135.95 68.02) (end 135.95 68.37) (width 0.5) (layer F.Cu) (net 8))
 (segment (start 135.21336 67.28336) (end 135.95 68.02) (width 0.5) (layer F.Cu) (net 8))
 (segment (start 135.97 68.05) (end 136.70664 67.31336) (width 0.5) (layer F.Cu) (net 8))
 (segment (start 136.49 67.37) (end 135.448234 67.37) (width 0.5) (layer F.Cu) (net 8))
 (segment (start 135.95 70.22) (end 135.949999 69.39) (width 0.5) (layer F.Cu) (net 9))
 (segment (start 137.88 74.07) (end 137.88 75.85) (width 0.5) (layer F.Cu) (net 13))
 (segment (start 135.95 72.14) (end 137.88 74.07) (width 0.5) (layer F.Cu) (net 13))
 (segment (start 135.95 72.12) (end 135.95 72.14) (width 0.5) (layer F.Cu) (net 13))
 (segment (start 141.64 70.75) (end 141.5 70.61) (width 0.25) (layer F.Cu) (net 7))
 (segment (start 141.64 71.604999) (end 141.64 70.75) (width 0.25) (layer F.Cu) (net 7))
 (segment (start 142.14 72.755) (end 142.14 73.65) (width 0.25) (layer F.Cu) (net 6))
 (segment (start 142.15 75.79) (end 142.15 73.72) (width 0.5) (layer F.Cu) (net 6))
 (segment (start 142.445 76.085) (end 142.15 75.79) (width 0.5) (layer F.Cu) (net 6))
 (segment (start 144.985 76.085) (end 142.445 76.085) (width 0.5) (layer F.Cu) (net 6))
 (segment (start 143.435 72.755) (end 143.51 72.68) (width 0.5) (layer F.Cu) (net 5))
 (segment (start 142.76 72.76) (end 143.555 72.76) (width 0.5) (layer F.Cu) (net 5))
 (segment (start 143.605 72.775) (end 144.985 72.775) (width 0.5) (layer F.Cu) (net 5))
 (segment (start 143.51 72.68) (end 143.605 72.775) (width 0.5) (layer F.Cu) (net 5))
 (segment (start 147.855 72.775) (end 147.854999 70.825) (width 0.5) (layer F.Cu) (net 12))
 (segment (start 147.855 76.085) (end 147.855 74.135) (width 0.5) (layer F.Cu) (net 12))
 (segment (start 147.855 72.775) (end 147.855 74.135) (width 0.5) (layer F.Cu) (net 12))
 (segment (start 147.63001 74.56001) (end 147.855 74.785) (width 0.5) (layer F.Cu) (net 12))
 (segment (start 147.63001 72.461468) (end 147.63001 74.56001) (width 0.5) (layer F.Cu) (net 12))
 (segment (start 147.855 72.686458) (end 147.63001 72.461468) (width 0.5) (layer F.Cu) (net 12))
 (segment (start 147.855 72.775) (end 147.855 72.686458) (width 0.5) (layer F.Cu) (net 12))
 (segment (start 147.52 72.775) (end 147.52 74.135) (width 0.5) (layer F.Cu) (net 12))
 (segment (start 132.39 71.17) (end 132.38 71.18) (width 0.5) (layer F.Cu) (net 1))
 (segment (start 133.75 71.170001) (end 132.39 71.17) (width 0.5) (layer F.Cu) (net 1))
 (segment (start 144.985 75.435) (end 144.984999 74.135) (width 0.5) (layer F.Cu) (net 1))
 (via (at 143.12 74.18) (size 0.4) (drill 0.3) (layers F.Cu B.Cu) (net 1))
 (via (at 143.12 74.92) (size 0.4) (drill 0.3) (layers F.Cu B.Cu) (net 1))
 (via (at 143.87 74.18) (size 0.4) (drill 0.3) (layers F.Cu B.Cu) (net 1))
 (via (at 143.87 74.92) (size 0.4) (drill 0.3) (layers F.Cu B.Cu) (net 1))
 (via (at 131.49 76.96) (size 0.4) (drill 0.3) (layers F.Cu B.Cu) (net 1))
 (via (at 131.49 76.22) (size 0.4) (drill 0.3) (layers F.Cu B.Cu) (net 1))
 (via (at 132.3 76.96) (size 0.4) (drill 0.3) (layers F.Cu B.Cu) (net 1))
 (via (at 133.05 76.22) (size 0.4) (drill 0.3) (layers F.Cu B.Cu) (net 1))
 (via (at 133.05 76.96) (size 0.4) (drill 0.3) (layers F.Cu B.Cu) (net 1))
 (via (at 132.3 76.22) (size 0.4) (drill 0.3) (layers F.Cu B.Cu) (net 1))
 (via (at 134.9 76.96) (size 0.4) (drill 0.3) (layers F.Cu B.Cu) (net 1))
 (via (at 134.15 76.96) (size 0.4) (drill 0.3) (layers F.Cu B.Cu) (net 1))
 (via (at 134.9 76.22) (size 0.4) (drill 0.3) (layers F.Cu B.Cu) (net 1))
 (via (at 134.15 76.22) (size 0.4) (drill 0.3) (layers F.Cu B.Cu) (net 1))
 (via (at 133.05 75.49) (size 0.4) (drill 0.3) (layers F.Cu B.Cu) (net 1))
 (via (at 131.49 75.49) (size 0.4) (drill 0.3) (layers F.Cu B.Cu) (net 1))
 (via (at 132.3 75.49) (size 0.4) (drill 0.3) (layers F.Cu B.Cu) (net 1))
 (via (at 134.9 75.49) (size 0.4) (drill 0.3) (layers F.Cu B.Cu) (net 1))
 (via (at 134.15 75.49) (size 0.4) (drill 0.3) (layers F.Cu B.Cu) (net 1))
 (via (at 132.37 72.069999) (size 0.4) (drill 0.3) (layers F.Cu B.Cu) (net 1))
 (via (at 131.62 72.07) (size 0.4) (drill 0.3) (layers F.Cu B.Cu) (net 1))
 (via (at 131.23 69.13) (size 0.4) (drill 0.3) (layers F.Cu B.Cu) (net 1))
 (via (at 131.98 69.129999) (size 0.4) (drill 0.3) (layers F.Cu B.Cu) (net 1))
 (via (at 131.98 68.359999) (size 0.4) (drill 0.3) (layers F.Cu B.Cu) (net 1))
 (via (at 131.23 68.36) (size 0.4) (drill 0.3) (layers F.Cu B.Cu) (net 1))
 (via (at 133.56 69.129999) (size 0.4) (drill 0.3) (layers F.Cu B.Cu) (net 1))
 (via (at 132.81 68.36) (size 0.4) (drill 0.3) (layers F.Cu B.Cu) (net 1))
 (via (at 132.81 69.13) (size 0.4) (drill 0.3) (layers F.Cu B.Cu) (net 1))
 (via (at 133.56 68.359999) (size 0.4) (drill 0.3) (layers F.Cu B.Cu) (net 1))
 (via (at 139.37 72.399999) (size 0.4) (drill 0.3) (layers F.Cu B.Cu) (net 1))
 (via (at 138.62 73.17) (size 0.4) (drill 0.3) (layers F.Cu B.Cu) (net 1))
 (via (at 139.37 73.169999) (size 0.4) (drill 0.3) (layers F.Cu B.Cu) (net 1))
 (via (at 138.62 72.4) (size 0.4) (drill 0.3) (layers F.Cu B.Cu) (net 1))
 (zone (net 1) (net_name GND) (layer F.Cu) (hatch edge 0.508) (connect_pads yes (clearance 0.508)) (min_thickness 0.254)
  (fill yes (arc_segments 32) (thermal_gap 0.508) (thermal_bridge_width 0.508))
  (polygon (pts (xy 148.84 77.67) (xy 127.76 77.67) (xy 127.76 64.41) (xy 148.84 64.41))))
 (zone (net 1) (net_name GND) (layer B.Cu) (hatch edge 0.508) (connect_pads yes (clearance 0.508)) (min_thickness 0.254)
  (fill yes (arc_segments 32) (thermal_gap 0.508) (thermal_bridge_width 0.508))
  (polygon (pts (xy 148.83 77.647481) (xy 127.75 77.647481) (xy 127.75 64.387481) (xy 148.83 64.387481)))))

